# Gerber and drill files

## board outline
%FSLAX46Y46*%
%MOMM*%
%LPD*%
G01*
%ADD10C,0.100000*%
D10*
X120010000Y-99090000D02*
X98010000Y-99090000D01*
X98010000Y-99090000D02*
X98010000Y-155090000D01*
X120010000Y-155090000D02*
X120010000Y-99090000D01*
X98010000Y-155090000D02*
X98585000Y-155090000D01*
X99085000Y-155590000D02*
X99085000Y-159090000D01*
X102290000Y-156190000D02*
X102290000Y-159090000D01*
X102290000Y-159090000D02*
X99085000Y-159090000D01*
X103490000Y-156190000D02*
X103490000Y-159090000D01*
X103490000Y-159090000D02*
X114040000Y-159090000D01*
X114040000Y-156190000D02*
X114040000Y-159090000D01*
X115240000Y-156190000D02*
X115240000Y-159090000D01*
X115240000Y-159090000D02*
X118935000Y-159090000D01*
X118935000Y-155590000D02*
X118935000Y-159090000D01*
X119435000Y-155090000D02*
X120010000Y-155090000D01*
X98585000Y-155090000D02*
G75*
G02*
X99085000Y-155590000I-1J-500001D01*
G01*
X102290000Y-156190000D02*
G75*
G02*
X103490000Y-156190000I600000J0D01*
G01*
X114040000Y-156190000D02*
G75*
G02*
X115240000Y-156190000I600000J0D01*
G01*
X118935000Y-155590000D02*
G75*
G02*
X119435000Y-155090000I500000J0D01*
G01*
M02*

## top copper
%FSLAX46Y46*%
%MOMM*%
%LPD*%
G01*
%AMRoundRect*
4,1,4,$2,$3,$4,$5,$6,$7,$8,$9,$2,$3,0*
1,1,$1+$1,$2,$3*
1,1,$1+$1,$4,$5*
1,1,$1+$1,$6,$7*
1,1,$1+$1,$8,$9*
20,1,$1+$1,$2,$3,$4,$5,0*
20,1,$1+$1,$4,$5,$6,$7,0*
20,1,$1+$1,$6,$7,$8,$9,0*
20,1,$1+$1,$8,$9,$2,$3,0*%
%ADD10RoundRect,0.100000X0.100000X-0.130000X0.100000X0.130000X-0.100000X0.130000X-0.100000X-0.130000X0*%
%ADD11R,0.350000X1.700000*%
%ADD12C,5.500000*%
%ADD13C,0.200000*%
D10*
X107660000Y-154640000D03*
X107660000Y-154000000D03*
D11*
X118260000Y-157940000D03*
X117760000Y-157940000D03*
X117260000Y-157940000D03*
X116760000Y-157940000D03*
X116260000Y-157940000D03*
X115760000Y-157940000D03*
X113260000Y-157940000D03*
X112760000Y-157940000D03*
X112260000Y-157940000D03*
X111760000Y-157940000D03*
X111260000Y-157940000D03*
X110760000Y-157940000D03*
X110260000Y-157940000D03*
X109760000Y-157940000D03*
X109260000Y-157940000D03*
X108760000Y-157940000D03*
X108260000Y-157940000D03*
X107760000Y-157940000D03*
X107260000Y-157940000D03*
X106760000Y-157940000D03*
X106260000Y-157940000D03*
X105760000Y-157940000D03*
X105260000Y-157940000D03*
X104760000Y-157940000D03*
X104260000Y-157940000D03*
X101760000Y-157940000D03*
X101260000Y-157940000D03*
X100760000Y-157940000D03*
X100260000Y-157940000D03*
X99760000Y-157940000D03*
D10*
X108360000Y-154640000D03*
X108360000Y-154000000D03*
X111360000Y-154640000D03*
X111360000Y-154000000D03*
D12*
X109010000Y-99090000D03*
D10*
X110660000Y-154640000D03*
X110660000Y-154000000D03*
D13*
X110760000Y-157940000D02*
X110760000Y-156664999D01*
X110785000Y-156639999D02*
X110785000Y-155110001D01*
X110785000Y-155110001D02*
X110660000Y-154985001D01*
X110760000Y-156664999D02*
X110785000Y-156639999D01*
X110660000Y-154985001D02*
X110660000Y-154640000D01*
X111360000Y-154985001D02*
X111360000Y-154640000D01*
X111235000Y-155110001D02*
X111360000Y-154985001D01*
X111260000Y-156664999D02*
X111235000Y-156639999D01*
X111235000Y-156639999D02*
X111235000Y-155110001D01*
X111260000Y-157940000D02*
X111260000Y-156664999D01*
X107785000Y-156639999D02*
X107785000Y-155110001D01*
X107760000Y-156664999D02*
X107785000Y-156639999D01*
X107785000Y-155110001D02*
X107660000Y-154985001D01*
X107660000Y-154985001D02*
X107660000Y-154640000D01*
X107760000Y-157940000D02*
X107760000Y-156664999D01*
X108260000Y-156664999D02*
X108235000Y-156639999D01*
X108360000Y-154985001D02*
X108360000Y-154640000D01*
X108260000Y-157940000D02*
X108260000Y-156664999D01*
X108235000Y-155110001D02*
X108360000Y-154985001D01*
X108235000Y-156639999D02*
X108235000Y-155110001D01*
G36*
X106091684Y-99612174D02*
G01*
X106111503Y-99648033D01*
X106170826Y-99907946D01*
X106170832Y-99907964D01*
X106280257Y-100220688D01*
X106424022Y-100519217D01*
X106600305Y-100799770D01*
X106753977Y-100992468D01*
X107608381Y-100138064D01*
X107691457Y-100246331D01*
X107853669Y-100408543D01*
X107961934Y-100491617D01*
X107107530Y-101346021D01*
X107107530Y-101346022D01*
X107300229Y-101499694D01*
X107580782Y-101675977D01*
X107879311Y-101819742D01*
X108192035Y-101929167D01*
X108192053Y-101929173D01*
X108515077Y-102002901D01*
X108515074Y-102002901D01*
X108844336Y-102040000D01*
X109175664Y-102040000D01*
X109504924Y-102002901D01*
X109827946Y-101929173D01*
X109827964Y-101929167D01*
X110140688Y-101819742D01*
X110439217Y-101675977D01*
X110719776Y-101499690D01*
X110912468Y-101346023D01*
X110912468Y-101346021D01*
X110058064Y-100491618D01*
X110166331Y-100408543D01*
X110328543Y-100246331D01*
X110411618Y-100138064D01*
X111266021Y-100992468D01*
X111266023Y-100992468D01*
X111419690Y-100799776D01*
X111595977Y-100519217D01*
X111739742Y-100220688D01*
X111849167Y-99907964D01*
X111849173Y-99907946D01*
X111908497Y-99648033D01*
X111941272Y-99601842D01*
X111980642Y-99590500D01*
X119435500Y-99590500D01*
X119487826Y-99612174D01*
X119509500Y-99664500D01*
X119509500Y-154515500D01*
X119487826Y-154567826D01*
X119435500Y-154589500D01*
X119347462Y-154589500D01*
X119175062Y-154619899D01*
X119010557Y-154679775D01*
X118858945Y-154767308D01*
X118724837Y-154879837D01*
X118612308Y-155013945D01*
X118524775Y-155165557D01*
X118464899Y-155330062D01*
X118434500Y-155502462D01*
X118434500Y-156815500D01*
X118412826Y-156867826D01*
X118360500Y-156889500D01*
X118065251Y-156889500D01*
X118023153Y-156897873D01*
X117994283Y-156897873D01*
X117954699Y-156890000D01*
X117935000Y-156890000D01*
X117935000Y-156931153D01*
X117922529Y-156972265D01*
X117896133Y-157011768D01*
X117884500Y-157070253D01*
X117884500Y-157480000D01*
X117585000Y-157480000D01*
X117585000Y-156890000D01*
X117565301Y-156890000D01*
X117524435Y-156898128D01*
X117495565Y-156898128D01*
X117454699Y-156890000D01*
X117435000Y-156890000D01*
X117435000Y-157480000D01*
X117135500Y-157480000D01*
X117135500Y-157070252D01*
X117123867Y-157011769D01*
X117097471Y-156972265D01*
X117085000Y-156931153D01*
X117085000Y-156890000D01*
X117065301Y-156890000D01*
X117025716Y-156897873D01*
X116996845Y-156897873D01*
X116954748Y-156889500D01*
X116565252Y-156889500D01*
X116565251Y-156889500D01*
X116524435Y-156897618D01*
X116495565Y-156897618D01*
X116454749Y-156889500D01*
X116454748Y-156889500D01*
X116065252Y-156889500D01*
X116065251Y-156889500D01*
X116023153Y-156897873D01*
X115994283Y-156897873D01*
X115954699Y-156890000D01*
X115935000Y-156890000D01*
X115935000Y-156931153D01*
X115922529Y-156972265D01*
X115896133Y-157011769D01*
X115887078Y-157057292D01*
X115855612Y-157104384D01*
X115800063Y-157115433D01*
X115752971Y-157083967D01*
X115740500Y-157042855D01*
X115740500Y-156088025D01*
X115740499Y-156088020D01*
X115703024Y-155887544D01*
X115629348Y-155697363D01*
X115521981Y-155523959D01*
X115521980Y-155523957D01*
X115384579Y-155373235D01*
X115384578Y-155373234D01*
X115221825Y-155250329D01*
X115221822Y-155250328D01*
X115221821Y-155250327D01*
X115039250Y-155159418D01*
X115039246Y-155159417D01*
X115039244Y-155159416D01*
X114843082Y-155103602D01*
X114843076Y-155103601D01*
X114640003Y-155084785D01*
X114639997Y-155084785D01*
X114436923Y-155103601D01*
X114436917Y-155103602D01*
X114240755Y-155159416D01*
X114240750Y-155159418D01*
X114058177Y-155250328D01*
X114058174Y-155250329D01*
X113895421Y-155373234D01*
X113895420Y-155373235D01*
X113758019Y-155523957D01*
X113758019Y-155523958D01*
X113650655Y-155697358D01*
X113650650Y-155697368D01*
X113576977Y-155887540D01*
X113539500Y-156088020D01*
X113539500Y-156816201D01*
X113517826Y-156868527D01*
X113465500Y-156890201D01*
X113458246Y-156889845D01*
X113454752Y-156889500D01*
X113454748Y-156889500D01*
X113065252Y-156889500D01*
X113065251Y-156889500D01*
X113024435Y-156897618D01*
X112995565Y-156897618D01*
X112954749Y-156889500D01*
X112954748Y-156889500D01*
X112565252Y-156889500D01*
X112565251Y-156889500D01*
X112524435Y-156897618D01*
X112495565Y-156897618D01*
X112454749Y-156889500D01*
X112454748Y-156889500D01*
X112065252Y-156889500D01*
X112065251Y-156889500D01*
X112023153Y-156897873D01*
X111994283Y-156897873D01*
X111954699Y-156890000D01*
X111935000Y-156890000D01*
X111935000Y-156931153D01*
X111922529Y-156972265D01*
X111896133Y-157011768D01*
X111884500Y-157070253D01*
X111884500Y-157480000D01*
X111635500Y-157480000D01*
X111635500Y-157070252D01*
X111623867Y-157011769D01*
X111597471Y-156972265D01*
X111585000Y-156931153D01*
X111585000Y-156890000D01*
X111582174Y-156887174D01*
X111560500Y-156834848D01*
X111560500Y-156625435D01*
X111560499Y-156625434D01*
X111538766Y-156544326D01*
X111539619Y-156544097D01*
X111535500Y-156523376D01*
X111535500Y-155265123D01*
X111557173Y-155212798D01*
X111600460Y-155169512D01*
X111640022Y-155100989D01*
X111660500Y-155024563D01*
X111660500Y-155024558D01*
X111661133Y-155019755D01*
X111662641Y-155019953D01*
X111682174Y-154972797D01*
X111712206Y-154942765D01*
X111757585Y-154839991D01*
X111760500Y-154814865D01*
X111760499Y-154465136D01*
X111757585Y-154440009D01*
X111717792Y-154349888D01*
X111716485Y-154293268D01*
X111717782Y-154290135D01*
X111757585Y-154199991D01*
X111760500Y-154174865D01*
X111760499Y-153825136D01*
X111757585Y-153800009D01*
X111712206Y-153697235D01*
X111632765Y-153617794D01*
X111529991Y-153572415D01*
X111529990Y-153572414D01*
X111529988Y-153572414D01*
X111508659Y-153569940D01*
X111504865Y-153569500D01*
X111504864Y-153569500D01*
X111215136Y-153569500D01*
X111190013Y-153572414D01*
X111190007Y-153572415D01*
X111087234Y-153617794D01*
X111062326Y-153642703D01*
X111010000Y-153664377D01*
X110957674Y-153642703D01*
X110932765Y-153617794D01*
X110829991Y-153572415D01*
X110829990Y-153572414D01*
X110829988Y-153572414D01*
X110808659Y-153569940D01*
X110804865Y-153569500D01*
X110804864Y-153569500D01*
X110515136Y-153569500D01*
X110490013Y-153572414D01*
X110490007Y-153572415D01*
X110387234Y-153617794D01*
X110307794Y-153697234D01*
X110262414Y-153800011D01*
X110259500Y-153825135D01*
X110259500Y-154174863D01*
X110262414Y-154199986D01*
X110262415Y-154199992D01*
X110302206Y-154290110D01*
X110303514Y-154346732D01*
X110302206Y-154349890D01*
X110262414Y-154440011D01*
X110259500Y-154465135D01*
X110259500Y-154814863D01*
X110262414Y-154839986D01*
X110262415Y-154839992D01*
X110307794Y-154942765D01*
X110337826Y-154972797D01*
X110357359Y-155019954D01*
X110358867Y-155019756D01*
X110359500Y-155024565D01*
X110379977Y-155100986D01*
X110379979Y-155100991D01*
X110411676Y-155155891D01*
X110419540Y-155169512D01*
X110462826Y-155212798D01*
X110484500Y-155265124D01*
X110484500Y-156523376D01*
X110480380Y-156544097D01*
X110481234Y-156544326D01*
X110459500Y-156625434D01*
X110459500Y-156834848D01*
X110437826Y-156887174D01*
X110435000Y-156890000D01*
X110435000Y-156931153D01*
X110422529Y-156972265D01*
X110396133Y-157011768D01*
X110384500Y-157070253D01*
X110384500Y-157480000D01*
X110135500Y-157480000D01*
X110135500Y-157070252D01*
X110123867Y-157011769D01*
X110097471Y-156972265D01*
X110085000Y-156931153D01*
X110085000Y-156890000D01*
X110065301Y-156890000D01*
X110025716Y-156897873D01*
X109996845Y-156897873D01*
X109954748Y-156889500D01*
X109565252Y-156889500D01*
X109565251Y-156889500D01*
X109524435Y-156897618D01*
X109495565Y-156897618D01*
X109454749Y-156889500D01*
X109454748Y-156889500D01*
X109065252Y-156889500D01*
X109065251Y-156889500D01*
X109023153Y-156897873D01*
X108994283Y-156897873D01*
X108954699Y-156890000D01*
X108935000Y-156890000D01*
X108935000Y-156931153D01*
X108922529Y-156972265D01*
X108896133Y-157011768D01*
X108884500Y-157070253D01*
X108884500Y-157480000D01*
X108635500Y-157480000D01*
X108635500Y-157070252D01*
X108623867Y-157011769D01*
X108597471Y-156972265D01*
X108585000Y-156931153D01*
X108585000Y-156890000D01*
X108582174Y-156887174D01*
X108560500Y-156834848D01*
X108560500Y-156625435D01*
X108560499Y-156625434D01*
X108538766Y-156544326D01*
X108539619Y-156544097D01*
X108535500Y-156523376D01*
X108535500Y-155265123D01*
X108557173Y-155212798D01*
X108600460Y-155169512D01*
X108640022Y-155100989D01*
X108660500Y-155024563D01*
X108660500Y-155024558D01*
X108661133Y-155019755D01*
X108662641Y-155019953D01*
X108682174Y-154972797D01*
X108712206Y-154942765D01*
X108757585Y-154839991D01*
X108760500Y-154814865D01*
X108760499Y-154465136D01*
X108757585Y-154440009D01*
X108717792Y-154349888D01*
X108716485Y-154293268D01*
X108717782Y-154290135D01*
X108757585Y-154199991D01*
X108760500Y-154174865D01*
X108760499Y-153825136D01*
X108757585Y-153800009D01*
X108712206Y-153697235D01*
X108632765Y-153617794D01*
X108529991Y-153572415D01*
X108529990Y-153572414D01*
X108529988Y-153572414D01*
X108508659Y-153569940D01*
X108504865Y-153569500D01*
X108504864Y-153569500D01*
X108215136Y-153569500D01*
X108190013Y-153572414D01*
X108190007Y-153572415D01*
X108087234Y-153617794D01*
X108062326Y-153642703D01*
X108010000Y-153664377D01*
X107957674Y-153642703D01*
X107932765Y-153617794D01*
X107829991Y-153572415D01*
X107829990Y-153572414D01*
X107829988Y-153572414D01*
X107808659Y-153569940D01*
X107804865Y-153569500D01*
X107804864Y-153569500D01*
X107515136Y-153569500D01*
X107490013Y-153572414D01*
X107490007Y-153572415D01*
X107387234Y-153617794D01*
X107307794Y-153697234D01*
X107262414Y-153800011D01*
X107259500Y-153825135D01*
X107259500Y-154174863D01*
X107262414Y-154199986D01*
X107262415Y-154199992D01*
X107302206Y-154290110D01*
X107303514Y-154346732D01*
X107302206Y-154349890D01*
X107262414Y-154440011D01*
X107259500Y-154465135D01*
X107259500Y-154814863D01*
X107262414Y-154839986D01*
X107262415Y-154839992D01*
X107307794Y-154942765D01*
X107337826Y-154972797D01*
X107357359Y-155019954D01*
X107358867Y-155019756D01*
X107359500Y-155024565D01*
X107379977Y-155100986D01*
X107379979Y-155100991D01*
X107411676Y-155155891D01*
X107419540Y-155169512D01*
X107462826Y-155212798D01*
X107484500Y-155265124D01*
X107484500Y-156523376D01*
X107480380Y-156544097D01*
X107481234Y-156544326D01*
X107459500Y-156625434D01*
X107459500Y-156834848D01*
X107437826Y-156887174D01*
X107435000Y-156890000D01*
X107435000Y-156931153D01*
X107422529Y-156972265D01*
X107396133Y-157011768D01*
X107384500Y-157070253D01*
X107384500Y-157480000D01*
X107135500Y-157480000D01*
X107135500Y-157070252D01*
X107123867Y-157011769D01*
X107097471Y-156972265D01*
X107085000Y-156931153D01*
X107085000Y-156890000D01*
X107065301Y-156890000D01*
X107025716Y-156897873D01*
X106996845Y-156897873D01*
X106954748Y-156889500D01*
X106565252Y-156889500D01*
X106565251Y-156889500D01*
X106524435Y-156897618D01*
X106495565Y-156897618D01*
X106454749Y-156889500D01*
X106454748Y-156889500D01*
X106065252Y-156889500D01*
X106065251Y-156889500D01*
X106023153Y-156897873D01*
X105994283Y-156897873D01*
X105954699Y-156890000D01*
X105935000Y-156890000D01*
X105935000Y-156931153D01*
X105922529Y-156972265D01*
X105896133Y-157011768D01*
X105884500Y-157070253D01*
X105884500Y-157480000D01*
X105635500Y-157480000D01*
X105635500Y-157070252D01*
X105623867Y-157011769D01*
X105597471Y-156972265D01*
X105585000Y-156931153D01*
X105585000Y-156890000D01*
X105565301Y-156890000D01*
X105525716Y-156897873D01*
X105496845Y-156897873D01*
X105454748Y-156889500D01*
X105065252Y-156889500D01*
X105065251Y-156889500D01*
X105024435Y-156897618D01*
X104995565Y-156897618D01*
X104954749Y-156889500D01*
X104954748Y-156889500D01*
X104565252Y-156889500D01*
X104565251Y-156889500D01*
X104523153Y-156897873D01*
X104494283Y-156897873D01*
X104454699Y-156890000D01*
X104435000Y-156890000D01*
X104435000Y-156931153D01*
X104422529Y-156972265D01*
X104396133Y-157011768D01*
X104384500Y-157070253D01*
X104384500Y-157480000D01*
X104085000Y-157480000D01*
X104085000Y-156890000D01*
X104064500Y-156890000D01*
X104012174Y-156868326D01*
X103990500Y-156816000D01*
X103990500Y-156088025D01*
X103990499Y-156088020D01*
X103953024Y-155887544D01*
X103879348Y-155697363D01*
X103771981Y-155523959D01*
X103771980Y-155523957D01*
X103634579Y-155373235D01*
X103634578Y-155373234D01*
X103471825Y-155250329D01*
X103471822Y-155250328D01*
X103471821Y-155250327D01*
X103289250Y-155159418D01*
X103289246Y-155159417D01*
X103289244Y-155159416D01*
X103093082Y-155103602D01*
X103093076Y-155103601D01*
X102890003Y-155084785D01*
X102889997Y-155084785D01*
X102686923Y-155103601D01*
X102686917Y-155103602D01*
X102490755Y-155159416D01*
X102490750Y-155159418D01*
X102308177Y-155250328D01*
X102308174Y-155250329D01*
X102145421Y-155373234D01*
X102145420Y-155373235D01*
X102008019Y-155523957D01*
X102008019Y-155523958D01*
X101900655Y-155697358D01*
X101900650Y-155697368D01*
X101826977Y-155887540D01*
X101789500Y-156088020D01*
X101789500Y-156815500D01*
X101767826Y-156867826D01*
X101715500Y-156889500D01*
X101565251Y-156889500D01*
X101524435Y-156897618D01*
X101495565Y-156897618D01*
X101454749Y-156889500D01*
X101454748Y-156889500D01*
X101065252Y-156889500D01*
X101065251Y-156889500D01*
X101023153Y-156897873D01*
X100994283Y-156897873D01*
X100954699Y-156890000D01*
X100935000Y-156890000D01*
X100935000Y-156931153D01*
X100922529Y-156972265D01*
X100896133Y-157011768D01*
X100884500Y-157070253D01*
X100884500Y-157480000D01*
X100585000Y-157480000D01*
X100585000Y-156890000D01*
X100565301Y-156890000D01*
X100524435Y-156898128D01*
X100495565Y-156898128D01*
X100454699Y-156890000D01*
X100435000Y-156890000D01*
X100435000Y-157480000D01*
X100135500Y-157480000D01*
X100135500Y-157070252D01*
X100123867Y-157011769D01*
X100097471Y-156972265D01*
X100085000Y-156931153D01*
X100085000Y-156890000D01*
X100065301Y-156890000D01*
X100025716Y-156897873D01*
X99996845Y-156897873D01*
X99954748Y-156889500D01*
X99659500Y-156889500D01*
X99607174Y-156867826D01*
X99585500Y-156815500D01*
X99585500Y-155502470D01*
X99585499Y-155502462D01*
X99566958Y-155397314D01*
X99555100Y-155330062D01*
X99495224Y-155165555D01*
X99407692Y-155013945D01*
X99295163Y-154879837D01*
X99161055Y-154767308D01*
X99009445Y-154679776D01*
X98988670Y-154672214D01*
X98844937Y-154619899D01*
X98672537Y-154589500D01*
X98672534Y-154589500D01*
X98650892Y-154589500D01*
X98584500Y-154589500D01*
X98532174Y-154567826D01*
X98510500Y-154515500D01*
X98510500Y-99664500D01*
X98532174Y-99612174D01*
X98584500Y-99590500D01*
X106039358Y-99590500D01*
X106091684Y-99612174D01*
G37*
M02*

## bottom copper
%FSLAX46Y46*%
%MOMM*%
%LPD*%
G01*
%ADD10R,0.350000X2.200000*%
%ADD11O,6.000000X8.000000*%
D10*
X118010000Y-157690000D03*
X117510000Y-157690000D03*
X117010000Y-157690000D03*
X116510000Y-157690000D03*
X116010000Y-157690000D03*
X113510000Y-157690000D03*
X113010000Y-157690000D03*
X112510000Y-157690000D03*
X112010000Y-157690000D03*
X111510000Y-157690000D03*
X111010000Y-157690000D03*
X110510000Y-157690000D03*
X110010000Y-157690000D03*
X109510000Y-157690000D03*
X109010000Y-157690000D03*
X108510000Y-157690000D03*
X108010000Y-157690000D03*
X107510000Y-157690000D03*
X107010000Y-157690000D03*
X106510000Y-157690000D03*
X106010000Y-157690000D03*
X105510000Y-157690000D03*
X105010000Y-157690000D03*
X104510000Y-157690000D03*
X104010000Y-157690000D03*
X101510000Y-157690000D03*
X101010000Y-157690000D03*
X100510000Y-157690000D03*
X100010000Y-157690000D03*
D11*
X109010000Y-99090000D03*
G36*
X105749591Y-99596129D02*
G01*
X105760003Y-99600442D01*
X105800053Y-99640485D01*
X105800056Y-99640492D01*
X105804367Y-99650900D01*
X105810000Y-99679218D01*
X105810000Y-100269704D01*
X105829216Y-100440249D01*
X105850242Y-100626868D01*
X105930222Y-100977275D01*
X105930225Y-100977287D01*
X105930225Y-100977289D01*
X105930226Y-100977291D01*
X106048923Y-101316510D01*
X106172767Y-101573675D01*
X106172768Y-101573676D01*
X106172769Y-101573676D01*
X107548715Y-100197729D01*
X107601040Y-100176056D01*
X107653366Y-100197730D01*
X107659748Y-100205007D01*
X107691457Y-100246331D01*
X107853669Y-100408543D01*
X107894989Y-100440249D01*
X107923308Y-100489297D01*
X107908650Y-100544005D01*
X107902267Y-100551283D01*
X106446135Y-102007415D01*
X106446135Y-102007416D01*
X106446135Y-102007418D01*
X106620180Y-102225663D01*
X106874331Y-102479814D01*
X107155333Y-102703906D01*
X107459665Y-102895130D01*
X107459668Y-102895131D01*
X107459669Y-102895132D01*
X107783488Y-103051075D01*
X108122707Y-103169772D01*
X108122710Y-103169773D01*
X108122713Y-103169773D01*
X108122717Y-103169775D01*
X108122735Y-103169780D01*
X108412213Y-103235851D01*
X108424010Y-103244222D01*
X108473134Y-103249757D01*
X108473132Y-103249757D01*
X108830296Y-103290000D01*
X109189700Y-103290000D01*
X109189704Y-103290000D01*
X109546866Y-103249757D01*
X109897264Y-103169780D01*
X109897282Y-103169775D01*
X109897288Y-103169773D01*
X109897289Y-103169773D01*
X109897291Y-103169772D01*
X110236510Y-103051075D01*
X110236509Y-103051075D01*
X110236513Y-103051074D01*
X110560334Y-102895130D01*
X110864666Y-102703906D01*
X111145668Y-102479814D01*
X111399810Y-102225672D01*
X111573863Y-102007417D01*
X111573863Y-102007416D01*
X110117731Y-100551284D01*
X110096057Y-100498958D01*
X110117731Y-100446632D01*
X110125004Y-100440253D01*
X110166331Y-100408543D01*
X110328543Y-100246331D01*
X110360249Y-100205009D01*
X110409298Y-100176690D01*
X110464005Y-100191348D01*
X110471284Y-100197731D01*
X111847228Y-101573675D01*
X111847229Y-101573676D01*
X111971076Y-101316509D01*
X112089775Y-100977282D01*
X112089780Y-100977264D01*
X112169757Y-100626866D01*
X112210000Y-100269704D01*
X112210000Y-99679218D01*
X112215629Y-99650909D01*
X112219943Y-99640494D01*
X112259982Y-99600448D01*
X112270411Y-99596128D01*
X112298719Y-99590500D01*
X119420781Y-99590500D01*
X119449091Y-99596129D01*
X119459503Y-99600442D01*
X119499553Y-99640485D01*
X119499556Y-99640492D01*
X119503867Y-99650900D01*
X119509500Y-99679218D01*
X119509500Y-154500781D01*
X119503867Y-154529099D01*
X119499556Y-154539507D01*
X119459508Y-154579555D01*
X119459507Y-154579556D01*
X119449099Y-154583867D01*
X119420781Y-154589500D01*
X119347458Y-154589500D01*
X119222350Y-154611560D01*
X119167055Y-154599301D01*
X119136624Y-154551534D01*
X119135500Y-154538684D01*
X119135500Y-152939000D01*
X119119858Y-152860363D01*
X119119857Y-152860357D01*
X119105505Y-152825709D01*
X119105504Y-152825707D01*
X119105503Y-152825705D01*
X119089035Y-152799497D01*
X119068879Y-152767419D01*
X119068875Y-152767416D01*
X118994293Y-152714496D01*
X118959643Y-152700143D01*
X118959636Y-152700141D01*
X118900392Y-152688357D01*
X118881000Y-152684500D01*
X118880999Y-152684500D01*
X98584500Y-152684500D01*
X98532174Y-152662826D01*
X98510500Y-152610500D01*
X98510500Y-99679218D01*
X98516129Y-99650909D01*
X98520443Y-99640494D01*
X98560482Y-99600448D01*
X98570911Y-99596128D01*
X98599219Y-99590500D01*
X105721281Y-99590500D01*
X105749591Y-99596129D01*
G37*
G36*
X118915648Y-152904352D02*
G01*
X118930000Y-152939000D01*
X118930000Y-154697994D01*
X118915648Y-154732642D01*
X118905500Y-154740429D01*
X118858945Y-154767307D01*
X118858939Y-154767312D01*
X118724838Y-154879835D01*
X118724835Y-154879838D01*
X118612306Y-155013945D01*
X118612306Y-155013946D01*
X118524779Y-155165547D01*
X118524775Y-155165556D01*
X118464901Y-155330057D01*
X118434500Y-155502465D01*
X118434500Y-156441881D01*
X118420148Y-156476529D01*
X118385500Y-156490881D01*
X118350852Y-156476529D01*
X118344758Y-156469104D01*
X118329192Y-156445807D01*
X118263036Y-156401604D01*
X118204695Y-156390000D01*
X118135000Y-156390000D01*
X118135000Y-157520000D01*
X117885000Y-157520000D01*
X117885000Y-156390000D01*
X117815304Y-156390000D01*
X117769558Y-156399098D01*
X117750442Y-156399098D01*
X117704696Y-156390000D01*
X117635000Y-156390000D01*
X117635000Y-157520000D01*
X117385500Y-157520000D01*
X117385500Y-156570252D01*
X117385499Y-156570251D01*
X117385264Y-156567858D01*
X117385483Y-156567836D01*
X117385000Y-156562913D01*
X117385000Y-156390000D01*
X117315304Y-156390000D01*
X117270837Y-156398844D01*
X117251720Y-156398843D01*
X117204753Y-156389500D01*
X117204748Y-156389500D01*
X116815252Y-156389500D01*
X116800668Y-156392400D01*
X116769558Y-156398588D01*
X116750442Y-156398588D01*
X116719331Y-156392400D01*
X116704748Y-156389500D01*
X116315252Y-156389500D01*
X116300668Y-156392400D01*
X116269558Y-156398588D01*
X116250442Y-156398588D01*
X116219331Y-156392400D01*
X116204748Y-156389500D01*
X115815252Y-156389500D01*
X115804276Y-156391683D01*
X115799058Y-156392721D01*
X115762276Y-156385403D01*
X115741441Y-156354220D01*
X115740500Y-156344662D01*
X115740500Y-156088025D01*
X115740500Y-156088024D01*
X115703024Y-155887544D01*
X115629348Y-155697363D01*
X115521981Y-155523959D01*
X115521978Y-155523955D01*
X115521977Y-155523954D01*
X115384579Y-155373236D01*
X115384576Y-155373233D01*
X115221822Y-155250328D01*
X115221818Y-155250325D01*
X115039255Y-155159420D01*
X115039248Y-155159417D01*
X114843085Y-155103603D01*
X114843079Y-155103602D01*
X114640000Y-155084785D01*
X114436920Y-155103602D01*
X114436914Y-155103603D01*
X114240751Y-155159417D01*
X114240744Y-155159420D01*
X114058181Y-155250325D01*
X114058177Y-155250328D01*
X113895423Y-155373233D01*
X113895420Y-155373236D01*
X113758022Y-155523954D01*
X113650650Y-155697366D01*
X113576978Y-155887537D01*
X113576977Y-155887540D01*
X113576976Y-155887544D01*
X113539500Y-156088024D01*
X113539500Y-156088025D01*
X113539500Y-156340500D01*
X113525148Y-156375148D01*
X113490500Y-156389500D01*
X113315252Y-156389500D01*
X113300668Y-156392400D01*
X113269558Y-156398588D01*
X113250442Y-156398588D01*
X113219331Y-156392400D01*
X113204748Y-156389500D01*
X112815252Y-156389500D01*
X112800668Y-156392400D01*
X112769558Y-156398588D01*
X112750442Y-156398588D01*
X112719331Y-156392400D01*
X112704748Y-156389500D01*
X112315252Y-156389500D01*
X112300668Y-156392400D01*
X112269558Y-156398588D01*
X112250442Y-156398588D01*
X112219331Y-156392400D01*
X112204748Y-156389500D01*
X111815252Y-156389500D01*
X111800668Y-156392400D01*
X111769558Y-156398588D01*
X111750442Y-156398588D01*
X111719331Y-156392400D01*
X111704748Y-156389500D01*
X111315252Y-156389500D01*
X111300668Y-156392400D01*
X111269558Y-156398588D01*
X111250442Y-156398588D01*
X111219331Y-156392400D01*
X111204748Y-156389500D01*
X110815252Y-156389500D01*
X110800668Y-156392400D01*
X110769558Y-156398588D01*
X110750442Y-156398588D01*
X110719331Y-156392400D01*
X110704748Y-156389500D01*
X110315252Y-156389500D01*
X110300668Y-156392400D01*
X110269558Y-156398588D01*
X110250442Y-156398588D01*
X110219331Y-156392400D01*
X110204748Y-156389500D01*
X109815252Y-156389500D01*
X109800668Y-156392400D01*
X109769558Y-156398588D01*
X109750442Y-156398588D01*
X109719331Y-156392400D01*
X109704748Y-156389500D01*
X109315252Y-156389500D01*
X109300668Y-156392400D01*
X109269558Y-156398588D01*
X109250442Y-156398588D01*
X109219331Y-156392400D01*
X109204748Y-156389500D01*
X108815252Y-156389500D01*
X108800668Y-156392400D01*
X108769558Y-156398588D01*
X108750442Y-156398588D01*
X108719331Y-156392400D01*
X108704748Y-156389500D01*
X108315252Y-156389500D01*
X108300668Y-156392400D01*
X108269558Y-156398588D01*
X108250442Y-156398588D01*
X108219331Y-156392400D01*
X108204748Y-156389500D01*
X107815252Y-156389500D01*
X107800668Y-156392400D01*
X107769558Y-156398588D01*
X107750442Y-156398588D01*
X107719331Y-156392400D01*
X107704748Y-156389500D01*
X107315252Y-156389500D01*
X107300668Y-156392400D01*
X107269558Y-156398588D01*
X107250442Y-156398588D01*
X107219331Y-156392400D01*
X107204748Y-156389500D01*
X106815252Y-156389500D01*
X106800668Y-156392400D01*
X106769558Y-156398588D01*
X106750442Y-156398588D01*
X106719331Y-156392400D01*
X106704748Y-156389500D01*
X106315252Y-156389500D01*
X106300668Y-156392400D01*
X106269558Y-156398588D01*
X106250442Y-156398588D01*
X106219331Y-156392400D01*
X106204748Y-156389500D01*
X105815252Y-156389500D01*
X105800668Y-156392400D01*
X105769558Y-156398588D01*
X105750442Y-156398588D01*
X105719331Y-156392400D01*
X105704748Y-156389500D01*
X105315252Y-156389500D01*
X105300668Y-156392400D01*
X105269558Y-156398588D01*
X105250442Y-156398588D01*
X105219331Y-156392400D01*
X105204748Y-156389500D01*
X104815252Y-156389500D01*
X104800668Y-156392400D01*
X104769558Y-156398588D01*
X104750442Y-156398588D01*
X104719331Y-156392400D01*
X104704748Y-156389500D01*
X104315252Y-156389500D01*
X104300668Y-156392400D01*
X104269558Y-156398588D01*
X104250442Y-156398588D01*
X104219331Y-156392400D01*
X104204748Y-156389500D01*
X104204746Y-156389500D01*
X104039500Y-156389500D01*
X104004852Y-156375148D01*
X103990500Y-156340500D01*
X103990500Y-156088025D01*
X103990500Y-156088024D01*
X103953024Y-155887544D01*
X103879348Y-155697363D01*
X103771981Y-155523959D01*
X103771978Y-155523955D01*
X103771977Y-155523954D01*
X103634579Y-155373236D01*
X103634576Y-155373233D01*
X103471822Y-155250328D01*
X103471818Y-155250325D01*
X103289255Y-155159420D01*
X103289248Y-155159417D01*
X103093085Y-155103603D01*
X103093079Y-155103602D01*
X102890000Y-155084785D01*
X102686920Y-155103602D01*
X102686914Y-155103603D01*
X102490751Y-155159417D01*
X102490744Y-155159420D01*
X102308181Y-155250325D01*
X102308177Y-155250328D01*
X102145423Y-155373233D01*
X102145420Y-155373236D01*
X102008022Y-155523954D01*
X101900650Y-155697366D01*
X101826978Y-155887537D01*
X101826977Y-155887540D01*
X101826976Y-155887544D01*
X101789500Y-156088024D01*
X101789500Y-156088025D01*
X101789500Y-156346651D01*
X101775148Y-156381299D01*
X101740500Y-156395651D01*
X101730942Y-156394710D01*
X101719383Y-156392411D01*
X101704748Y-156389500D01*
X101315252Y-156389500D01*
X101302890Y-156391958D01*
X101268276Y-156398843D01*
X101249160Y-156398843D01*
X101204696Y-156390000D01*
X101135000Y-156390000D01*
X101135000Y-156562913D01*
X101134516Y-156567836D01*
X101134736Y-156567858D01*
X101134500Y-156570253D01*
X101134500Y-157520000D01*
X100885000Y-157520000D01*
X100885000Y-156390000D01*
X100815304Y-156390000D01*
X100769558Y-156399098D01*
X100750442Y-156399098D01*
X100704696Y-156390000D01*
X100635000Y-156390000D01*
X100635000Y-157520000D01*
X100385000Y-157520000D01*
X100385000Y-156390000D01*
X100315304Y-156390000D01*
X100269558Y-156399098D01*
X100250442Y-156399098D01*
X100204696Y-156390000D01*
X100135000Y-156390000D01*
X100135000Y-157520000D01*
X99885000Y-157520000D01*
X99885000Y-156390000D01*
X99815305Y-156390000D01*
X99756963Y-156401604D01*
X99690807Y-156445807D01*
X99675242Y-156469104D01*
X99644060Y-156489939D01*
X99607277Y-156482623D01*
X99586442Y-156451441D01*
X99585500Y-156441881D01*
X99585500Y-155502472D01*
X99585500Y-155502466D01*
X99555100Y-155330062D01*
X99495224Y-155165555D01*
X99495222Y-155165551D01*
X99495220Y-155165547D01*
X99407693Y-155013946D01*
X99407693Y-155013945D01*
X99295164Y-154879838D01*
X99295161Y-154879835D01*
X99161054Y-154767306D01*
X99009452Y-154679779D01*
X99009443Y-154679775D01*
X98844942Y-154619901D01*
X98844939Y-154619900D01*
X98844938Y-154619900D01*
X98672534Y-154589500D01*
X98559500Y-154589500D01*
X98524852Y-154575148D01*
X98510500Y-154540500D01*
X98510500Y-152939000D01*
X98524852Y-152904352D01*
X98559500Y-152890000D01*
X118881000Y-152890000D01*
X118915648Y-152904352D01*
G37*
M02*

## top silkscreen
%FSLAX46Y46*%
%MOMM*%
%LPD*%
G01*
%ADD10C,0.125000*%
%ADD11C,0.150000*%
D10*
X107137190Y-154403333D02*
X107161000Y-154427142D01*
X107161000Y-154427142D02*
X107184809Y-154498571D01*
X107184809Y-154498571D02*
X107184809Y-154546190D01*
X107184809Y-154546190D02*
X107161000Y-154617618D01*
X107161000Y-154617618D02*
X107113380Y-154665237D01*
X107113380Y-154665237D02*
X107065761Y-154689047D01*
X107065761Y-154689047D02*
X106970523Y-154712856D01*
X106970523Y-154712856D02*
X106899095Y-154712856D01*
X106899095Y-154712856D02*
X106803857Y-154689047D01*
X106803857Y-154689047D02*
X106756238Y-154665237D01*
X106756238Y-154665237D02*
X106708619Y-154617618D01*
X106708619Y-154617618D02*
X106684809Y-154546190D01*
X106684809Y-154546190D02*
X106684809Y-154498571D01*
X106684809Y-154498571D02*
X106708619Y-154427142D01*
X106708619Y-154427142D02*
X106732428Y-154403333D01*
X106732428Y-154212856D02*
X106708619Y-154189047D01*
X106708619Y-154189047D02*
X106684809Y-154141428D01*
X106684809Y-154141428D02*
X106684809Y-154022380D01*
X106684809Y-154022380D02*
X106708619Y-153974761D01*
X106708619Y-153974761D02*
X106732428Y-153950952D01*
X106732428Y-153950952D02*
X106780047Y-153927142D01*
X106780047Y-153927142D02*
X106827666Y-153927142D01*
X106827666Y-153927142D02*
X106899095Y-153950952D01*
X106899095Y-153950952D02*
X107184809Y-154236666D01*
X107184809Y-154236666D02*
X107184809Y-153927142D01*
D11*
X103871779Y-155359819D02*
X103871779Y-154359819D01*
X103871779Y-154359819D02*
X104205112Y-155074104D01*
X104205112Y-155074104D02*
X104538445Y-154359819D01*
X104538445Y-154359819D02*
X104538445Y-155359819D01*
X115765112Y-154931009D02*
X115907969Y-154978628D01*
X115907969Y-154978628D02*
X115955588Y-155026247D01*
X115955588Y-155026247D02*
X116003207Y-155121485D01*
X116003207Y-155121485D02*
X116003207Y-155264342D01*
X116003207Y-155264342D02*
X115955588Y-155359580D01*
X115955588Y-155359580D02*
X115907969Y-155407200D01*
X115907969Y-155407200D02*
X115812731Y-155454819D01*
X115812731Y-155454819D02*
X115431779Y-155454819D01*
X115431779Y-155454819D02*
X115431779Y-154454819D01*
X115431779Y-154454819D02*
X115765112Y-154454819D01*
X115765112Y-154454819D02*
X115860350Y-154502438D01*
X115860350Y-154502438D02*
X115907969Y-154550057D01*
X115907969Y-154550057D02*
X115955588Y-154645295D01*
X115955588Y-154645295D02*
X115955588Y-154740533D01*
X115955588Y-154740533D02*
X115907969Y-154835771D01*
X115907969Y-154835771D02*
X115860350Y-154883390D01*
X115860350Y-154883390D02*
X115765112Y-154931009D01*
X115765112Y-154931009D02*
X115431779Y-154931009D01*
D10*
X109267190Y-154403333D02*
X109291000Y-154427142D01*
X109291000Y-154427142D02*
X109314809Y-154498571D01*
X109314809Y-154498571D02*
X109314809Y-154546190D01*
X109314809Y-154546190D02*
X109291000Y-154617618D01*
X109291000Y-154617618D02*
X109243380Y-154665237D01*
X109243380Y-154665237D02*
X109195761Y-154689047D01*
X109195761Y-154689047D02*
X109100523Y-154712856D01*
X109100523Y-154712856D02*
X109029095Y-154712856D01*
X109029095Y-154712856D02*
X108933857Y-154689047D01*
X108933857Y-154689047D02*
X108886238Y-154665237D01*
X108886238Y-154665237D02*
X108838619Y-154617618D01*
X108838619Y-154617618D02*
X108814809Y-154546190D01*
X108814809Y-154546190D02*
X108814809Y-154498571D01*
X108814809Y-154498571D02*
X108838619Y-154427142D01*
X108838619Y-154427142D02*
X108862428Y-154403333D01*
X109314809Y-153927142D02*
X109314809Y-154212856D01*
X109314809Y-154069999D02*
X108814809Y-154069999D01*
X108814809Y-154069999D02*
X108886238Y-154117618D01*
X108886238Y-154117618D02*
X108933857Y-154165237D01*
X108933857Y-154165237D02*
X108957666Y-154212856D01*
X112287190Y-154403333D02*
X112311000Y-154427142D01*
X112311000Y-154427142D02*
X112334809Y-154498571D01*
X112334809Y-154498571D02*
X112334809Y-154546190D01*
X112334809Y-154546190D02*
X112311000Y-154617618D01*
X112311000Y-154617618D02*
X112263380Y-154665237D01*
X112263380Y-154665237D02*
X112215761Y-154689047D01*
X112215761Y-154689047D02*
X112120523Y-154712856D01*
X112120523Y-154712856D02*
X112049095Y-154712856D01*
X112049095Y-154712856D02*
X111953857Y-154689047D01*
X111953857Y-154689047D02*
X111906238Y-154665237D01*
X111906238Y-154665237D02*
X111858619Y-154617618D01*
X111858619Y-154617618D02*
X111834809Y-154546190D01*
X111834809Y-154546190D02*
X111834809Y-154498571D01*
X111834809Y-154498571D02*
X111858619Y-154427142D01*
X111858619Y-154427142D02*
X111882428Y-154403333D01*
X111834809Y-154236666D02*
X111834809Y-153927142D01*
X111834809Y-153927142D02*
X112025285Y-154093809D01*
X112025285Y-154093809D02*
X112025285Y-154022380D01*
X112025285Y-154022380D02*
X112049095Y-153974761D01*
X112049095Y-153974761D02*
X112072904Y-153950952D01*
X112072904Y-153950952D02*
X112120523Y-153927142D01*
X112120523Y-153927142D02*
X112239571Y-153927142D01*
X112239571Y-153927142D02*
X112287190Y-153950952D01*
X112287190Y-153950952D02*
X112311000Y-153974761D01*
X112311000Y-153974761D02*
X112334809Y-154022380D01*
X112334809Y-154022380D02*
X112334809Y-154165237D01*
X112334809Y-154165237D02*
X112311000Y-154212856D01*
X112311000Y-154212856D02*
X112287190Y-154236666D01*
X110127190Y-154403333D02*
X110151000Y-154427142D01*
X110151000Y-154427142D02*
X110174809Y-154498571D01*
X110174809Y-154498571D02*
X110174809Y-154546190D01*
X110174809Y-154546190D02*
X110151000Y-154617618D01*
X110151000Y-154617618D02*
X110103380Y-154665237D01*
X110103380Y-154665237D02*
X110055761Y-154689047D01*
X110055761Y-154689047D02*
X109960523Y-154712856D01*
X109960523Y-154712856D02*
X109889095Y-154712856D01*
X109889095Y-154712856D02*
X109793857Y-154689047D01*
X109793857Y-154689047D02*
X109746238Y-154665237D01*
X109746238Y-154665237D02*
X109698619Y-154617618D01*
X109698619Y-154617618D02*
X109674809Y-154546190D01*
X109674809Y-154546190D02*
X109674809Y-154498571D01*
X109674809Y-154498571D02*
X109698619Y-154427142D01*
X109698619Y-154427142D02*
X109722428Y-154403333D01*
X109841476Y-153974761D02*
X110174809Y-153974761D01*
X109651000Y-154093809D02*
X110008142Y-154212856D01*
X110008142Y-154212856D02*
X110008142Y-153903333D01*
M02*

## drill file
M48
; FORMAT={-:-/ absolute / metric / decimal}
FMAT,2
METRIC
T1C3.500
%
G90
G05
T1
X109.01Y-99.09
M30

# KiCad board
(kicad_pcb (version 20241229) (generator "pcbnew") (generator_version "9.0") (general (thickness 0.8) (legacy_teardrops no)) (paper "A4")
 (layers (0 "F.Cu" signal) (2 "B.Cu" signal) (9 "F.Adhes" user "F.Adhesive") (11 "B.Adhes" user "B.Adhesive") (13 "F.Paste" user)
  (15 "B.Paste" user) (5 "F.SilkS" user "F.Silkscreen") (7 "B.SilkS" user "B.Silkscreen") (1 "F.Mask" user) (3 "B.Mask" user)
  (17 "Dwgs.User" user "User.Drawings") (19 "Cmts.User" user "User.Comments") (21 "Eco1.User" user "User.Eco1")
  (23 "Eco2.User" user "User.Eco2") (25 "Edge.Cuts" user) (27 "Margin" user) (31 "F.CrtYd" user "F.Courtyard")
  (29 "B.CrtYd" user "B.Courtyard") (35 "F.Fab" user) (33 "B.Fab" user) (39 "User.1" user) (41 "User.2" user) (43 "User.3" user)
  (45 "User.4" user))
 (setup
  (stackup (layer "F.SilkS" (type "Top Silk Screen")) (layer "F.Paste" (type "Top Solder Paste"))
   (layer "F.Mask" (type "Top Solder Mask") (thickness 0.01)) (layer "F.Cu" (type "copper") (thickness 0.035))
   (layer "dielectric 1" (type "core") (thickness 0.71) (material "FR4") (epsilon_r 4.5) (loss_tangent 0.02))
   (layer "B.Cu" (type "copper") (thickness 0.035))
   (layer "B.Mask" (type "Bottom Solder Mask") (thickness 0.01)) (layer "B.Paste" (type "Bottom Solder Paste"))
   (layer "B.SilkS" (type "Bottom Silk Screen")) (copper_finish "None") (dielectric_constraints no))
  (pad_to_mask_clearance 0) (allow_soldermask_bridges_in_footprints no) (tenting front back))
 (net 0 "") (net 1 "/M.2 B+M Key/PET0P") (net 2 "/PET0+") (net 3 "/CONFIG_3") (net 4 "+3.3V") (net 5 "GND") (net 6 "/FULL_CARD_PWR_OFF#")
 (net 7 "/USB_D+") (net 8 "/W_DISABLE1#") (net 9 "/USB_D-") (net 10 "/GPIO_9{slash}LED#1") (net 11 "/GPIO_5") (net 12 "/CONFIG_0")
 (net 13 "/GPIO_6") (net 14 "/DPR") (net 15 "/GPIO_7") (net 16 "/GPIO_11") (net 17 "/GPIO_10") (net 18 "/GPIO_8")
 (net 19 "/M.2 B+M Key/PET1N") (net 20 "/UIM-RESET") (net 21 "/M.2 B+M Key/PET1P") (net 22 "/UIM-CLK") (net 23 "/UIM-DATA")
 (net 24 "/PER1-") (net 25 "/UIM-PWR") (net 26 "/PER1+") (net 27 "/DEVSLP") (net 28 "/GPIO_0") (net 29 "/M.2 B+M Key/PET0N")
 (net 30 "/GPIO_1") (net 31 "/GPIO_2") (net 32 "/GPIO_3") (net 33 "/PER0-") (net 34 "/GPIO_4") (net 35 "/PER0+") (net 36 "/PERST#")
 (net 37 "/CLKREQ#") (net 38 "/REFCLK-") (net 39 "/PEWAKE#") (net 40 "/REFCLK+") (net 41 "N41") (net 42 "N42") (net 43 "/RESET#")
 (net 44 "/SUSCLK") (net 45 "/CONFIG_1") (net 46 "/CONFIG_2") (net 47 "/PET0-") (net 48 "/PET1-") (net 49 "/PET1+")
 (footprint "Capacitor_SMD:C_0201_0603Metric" (layer "F.Cu") (at 107.66 154.32 90)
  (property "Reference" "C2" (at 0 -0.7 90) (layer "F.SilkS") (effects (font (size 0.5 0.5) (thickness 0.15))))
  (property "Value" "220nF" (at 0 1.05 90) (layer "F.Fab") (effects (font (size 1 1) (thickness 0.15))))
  (pad "" smd roundrect (at -0.345 0 90) (size 0.318 0.36) (layers "F.Paste") (roundrect_rratio 0.25))
  (pad "" smd roundrect (at 0.345 0 90) (size 0.318 0.36) (layers "F.Paste") (roundrect_rratio 0.25))
  (pad "1" smd roundrect (at -0.32 0 90) (size 0.46 0.4) (layers "F.Cu" "F.Mask") (roundrect_rratio 0.25) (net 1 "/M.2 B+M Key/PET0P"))
  (pad "2" smd roundrect (at 0.32 0 90) (size 0.46 0.4) (layers "F.Cu" "F.Mask") (roundrect_rratio 0.25) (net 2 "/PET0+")))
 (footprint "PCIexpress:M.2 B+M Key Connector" (layer "F.Cu") (at 109.01 157.98)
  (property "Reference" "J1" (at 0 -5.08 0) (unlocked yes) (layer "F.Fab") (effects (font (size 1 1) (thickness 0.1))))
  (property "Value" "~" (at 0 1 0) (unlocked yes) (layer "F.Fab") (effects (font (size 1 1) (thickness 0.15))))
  (fp_line (start -11 -2.89) (end -10.425 -2.89) (stroke (width 0.1) (type default)) (layer "Edge.Cuts"))
  (fp_line (start -9.925 -2.39) (end -9.925 1.11) (stroke (width 0.1) (type default)) (layer "Edge.Cuts"))
  (fp_line (start -6.72 -1.79) (end -6.72 1.11) (stroke (width 0.1) (type default)) (layer "Edge.Cuts"))
  (fp_line (start -6.72 1.11) (end -9.925 1.11) (stroke (width 0.1) (type default)) (layer "Edge.Cuts"))
  (fp_line (start -5.52 -1.79) (end -5.52 1.11) (stroke (width 0.1) (type default)) (layer "Edge.Cuts"))
  (fp_line (start -5.52 1.11) (end 5.03 1.11) (stroke (width 0.1) (type default)) (layer "Edge.Cuts"))
  (fp_line (start 5.03 -1.79) (end 5.03 1.11) (stroke (width 0.1) (type default)) (layer "Edge.Cuts"))
  (fp_line (start 6.23 -1.79) (end 6.23 1.11) (stroke (width 0.1) (type default)) (layer "Edge.Cuts"))
  (fp_line (start 6.23 1.11) (end 9.925 1.11) (stroke (width 0.1) (type default)) (layer "Edge.Cuts"))
  (fp_line (start 9.925 -2.39) (end 9.925 1.11) (stroke (width 0.1) (type default)) (layer "Edge.Cuts"))
  (fp_line (start 10.425 -2.89) (end 11 -2.89) (stroke (width 0.1) (type default)) (layer "Edge.Cuts"))
  (fp_arc (start -10.425 -2.89) (mid -10.071447 -2.743553) (end -9.925 -2.39) (stroke (width 0.1) (type default)) (layer "Edge.Cuts"))
  (fp_arc (start -6.72 -1.79) (mid -6.12 -2.39) (end -5.52 -1.79) (stroke (width 0.1) (type default)) (layer "Edge.Cuts"))
  (fp_arc (start 5.03 -1.79) (mid 5.63 -2.39) (end 6.23 -1.79) (stroke (width 0.1) (type default)) (layer "Edge.Cuts"))
  (fp_arc (start 9.925 -2.39) (mid 10.071447 -2.743553) (end 10.425 -2.89) (stroke (width 0.1) (type default)) (layer "Edge.Cuts"))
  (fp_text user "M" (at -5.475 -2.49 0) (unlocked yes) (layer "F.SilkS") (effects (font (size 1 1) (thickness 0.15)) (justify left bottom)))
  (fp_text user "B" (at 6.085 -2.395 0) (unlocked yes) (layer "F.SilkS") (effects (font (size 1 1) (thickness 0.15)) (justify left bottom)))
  (pad "1" smd rect (at 9.25 -0.04 180) (size 0.35 1.7) (layers "F.Cu") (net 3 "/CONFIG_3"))
  (pad "2" smd rect (at 9 -0.29 180) (size 0.35 2.2) (layers "B.Cu") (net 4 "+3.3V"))
  (pad "3" smd rect (at 8.75 -0.04 180) (size 0.35 1.7) (layers "F.Cu") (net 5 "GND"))
  (pad "4" smd rect (at 8.5 -0.29 180) (size 0.35 2.2) (layers "B.Cu") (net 4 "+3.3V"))
  (pad "5" smd rect (at 8.25 -0.04 180) (size 0.35 1.7) (layers "F.Cu") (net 5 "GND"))
  (pad "6" smd rect (at 8 -0.29 180) (size 0.35 2.2) (layers "B.Cu") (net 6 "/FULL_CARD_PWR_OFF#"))
  (pad "7" smd rect (at 7.75 -0.04 180) (size 0.35 1.7) (layers "F.Cu") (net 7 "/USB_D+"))
  (pad "8" smd rect (at 7.5 -0.29 180) (size 0.35 2.2) (layers "B.Cu") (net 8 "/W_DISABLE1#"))
  (pad "9" smd rect (at 7.25 -0.04 180) (size 0.35 1.7) (layers "F.Cu") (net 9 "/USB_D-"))
  (pad "10" smd rect (at 7 -0.29 180) (size 0.35 2.2) (layers "B.Cu") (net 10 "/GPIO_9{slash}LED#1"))
  (pad "11" smd rect (at 6.75 -0.04 180) (size 0.35 1.7) (layers "F.Cu") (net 5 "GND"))
  (pad "20" smd rect (at 4.5 -0.29 180) (size 0.35 2.2) (layers "B.Cu") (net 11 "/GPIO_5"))
  (pad "21" smd rect (at 4.25 -0.04 180) (size 0.35 1.7) (layers "F.Cu") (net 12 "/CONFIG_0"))
  (pad "22" smd rect (at 4 -0.29 180) (size 0.35 2.2) (layers "B.Cu") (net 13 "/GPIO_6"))
  (pad "23" smd rect (at 3.75 -0.04 180) (size 0.35 1.7) (layers "F.Cu") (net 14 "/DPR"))
  (pad "24" smd rect (at 3.5 -0.29 180) (size 0.35 2.2) (layers "B.Cu") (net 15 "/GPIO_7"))
  (pad "25" smd rect (at 3.25 -0.04 180) (size 0.35 1.7) (layers "F.Cu") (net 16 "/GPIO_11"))
  (pad "26" smd rect (at 3 -0.29 180) (size 0.35 2.2) (layers "B.Cu") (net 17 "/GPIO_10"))
  (pad "27" smd rect (at 2.75 -0.04 180) (size 0.35 1.7) (layers "F.Cu") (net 5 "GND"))
  (pad "28" smd rect (at 2.5 -0.29 180) (size 0.35 2.2) (layers "B.Cu") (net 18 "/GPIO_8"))
  (pad "29" smd rect (at 2.25 -0.04 180) (size 0.35 1.7) (layers "F.Cu") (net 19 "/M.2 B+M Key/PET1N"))
  (pad "30" smd rect (at 2 -0.29 180) (size 0.35 2.2) (layers "B.Cu") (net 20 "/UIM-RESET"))
  (pad "31" smd rect (at 1.75 -0.04 180) (size 0.35 1.7) (layers "F.Cu") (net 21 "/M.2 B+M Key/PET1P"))
  (pad "32" smd rect (at 1.5 -0.29 180) (size 0.35 2.2) (layers "B.Cu") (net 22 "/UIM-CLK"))
  (pad "33" smd rect (at 1.25 -0.04 180) (size 0.35 1.7) (layers "F.Cu") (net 5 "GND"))
  (pad "34" smd rect (at 1 -0.29 180) (size 0.35 2.2) (layers "B.Cu") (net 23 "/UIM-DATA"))
  (pad "35" smd rect (at 0.75 -0.04 180) (size 0.35 1.7) (layers "F.Cu") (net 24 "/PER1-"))
  (pad "36" smd rect (at 0.5 -0.29 180) (size 0.35 2.2) (layers "B.Cu") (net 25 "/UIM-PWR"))
  (pad "37" smd rect (at 0.25 -0.04 180) (size 0.35 1.7) (layers "F.Cu") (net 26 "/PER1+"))
  (pad "38" smd rect (at 0 -0.29 180) (size 0.35 2.2) (layers "B.Cu") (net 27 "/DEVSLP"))
  (pad "39" smd rect (at -0.25 -0.04 180) (size 0.35 1.7) (layers "F.Cu") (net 5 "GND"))
  (pad "40" smd rect (at -0.5 -0.29 180) (size 0.35 2.2) (layers "B.Cu") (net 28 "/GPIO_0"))
  (pad "41" smd rect (at -0.75 -0.04 180) (size 0.35 1.7) (layers "F.Cu") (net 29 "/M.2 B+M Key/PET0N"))
  (pad "42" smd rect (at -1 -0.29 180) (size 0.35 2.2) (layers "B.Cu") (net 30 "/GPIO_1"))
  (pad "43" smd rect (at -1.25 -0.04 180) (size 0.35 1.7) (layers "F.Cu") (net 1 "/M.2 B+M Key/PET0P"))
  (pad "44" smd rect (at -1.5 -0.29 180) (size 0.35 2.2) (layers "B.Cu") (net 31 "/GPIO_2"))
  (pad "45" smd rect (at -1.75 -0.04 180) (size 0.35 1.7) (layers "F.Cu") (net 5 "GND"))
  (pad "46" smd rect (at -2 -0.29 180) (size 0.35 2.2) (layers "B.Cu") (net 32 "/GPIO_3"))
  (pad "47" smd rect (at -2.25 -0.04 180) (size 0.35 1.7) (layers "F.Cu") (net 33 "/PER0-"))
  (pad "48" smd rect (at -2.5 -0.29 180) (size 0.35 2.2) (layers "B.Cu") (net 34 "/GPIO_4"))
  (pad "49" smd rect (at -2.75 -0.04 180) (size 0.35 1.7) (layers "F.Cu") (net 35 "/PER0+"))
  (pad "50" smd rect (at -3 -0.29 180) (size 0.35 2.2) (layers "B.Cu") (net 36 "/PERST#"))
  (pad "51" smd rect (at -3.25 -0.04 180) (size 0.35 1.7) (layers "F.Cu") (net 5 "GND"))
  (pad "52" smd rect (at -3.5 -0.29 180) (size 0.35 2.2) (layers "B.Cu") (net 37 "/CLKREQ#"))
  (pad "53" smd rect (at -3.75 -0.04 180) (size 0.35 1.7) (layers "F.Cu") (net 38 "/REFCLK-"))
  (pad "54" smd rect (at -4 -0.29 180) (size 0.35 2.2) (layers "B.Cu") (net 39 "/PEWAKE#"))
  (pad "55" smd rect (at -4.25 -0.04 180) (size 0.35 1.7) (layers "F.Cu") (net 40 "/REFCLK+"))
  (pad "56" smd rect (at -4.5 -0.29 180) (size 0.35 2.2) (layers "B.Cu") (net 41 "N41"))
  (pad "57" smd rect (at -4.75 -0.04 180) (size 0.35 1.7) (layers "F.Cu") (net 5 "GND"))
  (pad "58" smd rect (at -5 -0.29 180) (size 0.35 2.2) (layers "B.Cu") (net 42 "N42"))
  (pad "67" smd rect (at -7.25 -0.04 180) (size 0.35 1.7) (layers "F.Cu") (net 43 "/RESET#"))
  (pad "68" smd rect (at -7.5 -0.29 180) (size 0.35 2.2) (layers "B.Cu") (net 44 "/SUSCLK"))
  (pad "69" smd rect (at -7.75 -0.04 180) (size 0.35 1.7) (layers "F.Cu") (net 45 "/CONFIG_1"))
  (pad "70" smd rect (at -8 -0.29 180) (size 0.35 2.2) (layers "B.Cu") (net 4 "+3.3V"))
  (pad "71" smd rect (at -8.25 -0.04 180) (size 0.35 1.7) (layers "F.Cu") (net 5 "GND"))
  (pad "72" smd rect (at -8.5 -0.29 180) (size 0.35 2.2) (layers "B.Cu") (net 4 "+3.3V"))
  (pad "73" smd rect (at -8.75 -0.04 180) (size 0.35 1.7) (layers "F.Cu") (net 5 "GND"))
  (pad "74" smd rect (at -9 -0.29 180) (size 0.35 2.2) (layers "B.Cu") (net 4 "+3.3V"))
  (pad "75" smd rect (at -9.25 -0.04 180) (size 0.35 1.7) (layers "F.Cu") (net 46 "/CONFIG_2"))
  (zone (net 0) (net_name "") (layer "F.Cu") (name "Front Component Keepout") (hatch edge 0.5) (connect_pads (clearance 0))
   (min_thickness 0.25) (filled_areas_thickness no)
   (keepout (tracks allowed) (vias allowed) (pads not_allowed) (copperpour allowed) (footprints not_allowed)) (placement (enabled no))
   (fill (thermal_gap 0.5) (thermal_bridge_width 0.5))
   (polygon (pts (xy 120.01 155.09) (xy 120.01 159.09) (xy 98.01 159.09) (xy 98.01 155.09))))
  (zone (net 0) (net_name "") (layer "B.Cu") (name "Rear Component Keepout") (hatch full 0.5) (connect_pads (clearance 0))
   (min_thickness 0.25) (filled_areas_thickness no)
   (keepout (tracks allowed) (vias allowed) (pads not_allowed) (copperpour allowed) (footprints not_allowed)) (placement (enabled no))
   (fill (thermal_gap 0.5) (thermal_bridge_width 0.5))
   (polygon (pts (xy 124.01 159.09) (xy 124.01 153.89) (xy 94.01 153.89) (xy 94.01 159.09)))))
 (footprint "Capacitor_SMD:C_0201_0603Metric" (layer "F.Cu") (at 108.36 154.32 90)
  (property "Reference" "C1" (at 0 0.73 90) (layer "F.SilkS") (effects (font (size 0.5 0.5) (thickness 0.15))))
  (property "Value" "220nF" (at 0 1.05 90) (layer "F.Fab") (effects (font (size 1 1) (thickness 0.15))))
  (pad "" smd roundrect (at -0.345 0 90) (size 0.318 0.36) (layers "F.Paste") (roundrect_rratio 0.25))
  (pad "" smd roundrect (at 0.345 0 90) (size 0.318 0.36) (layers "F.Paste") (roundrect_rratio 0.25))
  (pad "1" smd roundrect (at -0.32 0 90) (size 0.46 0.4) (layers "F.Cu" "F.Mask") (roundrect_rratio 0.25) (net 29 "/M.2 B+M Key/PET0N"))
  (pad "2" smd roundrect (at 0.32 0 90) (size 0.46 0.4) (layers "F.Cu" "F.Mask") (roundrect_rratio 0.25) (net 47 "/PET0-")))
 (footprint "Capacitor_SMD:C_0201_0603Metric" (layer "F.Cu") (at 111.36 154.32 90)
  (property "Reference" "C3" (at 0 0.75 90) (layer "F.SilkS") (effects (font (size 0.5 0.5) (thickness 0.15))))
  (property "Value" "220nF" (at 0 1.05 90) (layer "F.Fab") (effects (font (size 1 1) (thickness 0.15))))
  (pad "" smd roundrect (at -0.345 0 90) (size 0.318 0.36) (layers "F.Paste") (roundrect_rratio 0.25))
  (pad "" smd roundrect (at 0.345 0 90) (size 0.318 0.36) (layers "F.Paste") (roundrect_rratio 0.25))
  (pad "1" smd roundrect (at -0.32 0 90) (size 0.46 0.4) (layers "F.Cu" "F.Mask") (roundrect_rratio 0.25) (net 19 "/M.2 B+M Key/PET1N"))
  (pad "2" smd roundrect (at 0.32 0 90) (size 0.46 0.4) (layers "F.Cu" "F.Mask") (roundrect_rratio 0.25) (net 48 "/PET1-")))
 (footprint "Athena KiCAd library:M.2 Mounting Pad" (layer "F.Cu") (at 109.01 99.09)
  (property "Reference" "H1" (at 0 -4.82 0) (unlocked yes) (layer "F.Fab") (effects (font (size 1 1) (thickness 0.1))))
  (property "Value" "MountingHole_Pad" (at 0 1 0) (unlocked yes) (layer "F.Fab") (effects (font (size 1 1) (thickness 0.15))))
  (pad "1" thru_hole circle (at 0 0) (size 5.5 5.5) (drill 3.5) (layers "*.Cu" "*.Mask") (remove_unused_layers no) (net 5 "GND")
   (padstack (mode front_inner_back)
    (layer "Inner" (shape circle) (size 5.5 5.5) (zone_connect -1))
    (layer "B.Cu" (shape oval) (size 6 8) (thermal_bridge_angle 45) (zone_connect -1)))))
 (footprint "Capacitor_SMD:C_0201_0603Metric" (layer "F.Cu") (at 110.66 154.32 90)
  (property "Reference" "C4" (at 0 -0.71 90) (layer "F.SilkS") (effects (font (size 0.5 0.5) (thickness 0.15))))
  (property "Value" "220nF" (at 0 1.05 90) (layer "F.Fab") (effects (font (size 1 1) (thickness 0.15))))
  (pad "" smd roundrect (at -0.345 0 90) (size 0.318 0.36) (layers "F.Paste") (roundrect_rratio 0.25))
  (pad "" smd roundrect (at 0.345 0 90) (size 0.318 0.36) (layers "F.Paste") (roundrect_rratio 0.25))
  (pad "1" smd roundrect (at -0.32 0 90) (size 0.46 0.4) (layers "F.Cu" "F.Mask") (roundrect_rratio 0.25) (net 21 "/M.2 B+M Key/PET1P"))
  (pad "2" smd roundrect (at 0.32 0 90) (size 0.46 0.4) (layers "F.Cu" "F.Mask") (roundrect_rratio 0.25) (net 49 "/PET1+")))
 (gr_line (start 120.01 99.09) (end 98.01 99.09) (stroke (width 0.1) (type default)) (layer "Edge.Cuts"))
 (gr_line (start 98.01 99.09) (end 98.01 155.09) (stroke (width 0.1) (type default)) (layer "Edge.Cuts"))
 (gr_line (start 120.01 155.09) (end 120.01 99.09) (stroke (width 0.1) (type default)) (layer "Edge.Cuts"))
 (segment (start 110.76 157.94) (end 110.76 156.664999) (width 0.2) (layer "F.Cu") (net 21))
 (segment (start 110.785 156.639999) (end 110.785 155.110001) (width 0.2) (layer "F.Cu") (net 21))
 (segment (start 110.785 155.110001) (end 110.66 154.985001) (width 0.2) (layer "F.Cu") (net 21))
 (segment (start 110.76 156.664999) (end 110.785 156.639999) (width 0.2) (layer "F.Cu") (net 21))
 (segment (start 110.66 154.985001) (end 110.66 154.64) (width 0.2) (layer "F.Cu") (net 21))
 (segment (start 111.36 154.985001) (end 111.36 154.64) (width 0.2) (layer "F.Cu") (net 19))
 (segment (start 111.235 155.110001) (end 111.36 154.985001) (width 0.2) (layer "F.Cu") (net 19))
 (segment (start 111.26 156.664999) (end 111.235 156.639999) (width 0.2) (layer "F.Cu") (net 19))
 (segment (start 111.235 156.639999) (end 111.235 155.110001) (width 0.2) (layer "F.Cu") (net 19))
 (segment (start 111.26 157.94) (end 111.26 156.664999) (width 0.2) (layer "F.Cu") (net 19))
 (segment (start 107.785 156.639999) (end 107.785 155.110001) (width 0.2) (layer "F.Cu") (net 1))
 (segment (start 107.76 156.664999) (end 107.785 156.639999) (width 0.2) (layer "F.Cu") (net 1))
 (segment (start 107.785 155.110001) (end 107.66 154.985001) (width 0.2) (layer "F.Cu") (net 1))
 (segment (start 107.66 154.985001) (end 107.66 154.64) (width 0.2) (layer "F.Cu") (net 1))
 (segment (start 107.76 157.94) (end 107.76 156.664999) (width 0.2) (layer "F.Cu") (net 1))
 (segment (start 108.26 156.664999) (end 108.235 156.639999) (width 0.2) (layer "F.Cu") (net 29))
 (segment (start 108.36 154.985001) (end 108.36 154.64) (width 0.2) (layer "F.Cu") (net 29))
 (segment (start 108.26 157.94) (end 108.26 156.664999) (width 0.2) (layer "F.Cu") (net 29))
 (segment (start 108.235 155.110001) (end 108.36 154.985001) (width 0.2) (layer "F.Cu") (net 29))
 (segment (start 108.235 156.639999) (end 108.235 155.110001) (width 0.2) (layer "F.Cu") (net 29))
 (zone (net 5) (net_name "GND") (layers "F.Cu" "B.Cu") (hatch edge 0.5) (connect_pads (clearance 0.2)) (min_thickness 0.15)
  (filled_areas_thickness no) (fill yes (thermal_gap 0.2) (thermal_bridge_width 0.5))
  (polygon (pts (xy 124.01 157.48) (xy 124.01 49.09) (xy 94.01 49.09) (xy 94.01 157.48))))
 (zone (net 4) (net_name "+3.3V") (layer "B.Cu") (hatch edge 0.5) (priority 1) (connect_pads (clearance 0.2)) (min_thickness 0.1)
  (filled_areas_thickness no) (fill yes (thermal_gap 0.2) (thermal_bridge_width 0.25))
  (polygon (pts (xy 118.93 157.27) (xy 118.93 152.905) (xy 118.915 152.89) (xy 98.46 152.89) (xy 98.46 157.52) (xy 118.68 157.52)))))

